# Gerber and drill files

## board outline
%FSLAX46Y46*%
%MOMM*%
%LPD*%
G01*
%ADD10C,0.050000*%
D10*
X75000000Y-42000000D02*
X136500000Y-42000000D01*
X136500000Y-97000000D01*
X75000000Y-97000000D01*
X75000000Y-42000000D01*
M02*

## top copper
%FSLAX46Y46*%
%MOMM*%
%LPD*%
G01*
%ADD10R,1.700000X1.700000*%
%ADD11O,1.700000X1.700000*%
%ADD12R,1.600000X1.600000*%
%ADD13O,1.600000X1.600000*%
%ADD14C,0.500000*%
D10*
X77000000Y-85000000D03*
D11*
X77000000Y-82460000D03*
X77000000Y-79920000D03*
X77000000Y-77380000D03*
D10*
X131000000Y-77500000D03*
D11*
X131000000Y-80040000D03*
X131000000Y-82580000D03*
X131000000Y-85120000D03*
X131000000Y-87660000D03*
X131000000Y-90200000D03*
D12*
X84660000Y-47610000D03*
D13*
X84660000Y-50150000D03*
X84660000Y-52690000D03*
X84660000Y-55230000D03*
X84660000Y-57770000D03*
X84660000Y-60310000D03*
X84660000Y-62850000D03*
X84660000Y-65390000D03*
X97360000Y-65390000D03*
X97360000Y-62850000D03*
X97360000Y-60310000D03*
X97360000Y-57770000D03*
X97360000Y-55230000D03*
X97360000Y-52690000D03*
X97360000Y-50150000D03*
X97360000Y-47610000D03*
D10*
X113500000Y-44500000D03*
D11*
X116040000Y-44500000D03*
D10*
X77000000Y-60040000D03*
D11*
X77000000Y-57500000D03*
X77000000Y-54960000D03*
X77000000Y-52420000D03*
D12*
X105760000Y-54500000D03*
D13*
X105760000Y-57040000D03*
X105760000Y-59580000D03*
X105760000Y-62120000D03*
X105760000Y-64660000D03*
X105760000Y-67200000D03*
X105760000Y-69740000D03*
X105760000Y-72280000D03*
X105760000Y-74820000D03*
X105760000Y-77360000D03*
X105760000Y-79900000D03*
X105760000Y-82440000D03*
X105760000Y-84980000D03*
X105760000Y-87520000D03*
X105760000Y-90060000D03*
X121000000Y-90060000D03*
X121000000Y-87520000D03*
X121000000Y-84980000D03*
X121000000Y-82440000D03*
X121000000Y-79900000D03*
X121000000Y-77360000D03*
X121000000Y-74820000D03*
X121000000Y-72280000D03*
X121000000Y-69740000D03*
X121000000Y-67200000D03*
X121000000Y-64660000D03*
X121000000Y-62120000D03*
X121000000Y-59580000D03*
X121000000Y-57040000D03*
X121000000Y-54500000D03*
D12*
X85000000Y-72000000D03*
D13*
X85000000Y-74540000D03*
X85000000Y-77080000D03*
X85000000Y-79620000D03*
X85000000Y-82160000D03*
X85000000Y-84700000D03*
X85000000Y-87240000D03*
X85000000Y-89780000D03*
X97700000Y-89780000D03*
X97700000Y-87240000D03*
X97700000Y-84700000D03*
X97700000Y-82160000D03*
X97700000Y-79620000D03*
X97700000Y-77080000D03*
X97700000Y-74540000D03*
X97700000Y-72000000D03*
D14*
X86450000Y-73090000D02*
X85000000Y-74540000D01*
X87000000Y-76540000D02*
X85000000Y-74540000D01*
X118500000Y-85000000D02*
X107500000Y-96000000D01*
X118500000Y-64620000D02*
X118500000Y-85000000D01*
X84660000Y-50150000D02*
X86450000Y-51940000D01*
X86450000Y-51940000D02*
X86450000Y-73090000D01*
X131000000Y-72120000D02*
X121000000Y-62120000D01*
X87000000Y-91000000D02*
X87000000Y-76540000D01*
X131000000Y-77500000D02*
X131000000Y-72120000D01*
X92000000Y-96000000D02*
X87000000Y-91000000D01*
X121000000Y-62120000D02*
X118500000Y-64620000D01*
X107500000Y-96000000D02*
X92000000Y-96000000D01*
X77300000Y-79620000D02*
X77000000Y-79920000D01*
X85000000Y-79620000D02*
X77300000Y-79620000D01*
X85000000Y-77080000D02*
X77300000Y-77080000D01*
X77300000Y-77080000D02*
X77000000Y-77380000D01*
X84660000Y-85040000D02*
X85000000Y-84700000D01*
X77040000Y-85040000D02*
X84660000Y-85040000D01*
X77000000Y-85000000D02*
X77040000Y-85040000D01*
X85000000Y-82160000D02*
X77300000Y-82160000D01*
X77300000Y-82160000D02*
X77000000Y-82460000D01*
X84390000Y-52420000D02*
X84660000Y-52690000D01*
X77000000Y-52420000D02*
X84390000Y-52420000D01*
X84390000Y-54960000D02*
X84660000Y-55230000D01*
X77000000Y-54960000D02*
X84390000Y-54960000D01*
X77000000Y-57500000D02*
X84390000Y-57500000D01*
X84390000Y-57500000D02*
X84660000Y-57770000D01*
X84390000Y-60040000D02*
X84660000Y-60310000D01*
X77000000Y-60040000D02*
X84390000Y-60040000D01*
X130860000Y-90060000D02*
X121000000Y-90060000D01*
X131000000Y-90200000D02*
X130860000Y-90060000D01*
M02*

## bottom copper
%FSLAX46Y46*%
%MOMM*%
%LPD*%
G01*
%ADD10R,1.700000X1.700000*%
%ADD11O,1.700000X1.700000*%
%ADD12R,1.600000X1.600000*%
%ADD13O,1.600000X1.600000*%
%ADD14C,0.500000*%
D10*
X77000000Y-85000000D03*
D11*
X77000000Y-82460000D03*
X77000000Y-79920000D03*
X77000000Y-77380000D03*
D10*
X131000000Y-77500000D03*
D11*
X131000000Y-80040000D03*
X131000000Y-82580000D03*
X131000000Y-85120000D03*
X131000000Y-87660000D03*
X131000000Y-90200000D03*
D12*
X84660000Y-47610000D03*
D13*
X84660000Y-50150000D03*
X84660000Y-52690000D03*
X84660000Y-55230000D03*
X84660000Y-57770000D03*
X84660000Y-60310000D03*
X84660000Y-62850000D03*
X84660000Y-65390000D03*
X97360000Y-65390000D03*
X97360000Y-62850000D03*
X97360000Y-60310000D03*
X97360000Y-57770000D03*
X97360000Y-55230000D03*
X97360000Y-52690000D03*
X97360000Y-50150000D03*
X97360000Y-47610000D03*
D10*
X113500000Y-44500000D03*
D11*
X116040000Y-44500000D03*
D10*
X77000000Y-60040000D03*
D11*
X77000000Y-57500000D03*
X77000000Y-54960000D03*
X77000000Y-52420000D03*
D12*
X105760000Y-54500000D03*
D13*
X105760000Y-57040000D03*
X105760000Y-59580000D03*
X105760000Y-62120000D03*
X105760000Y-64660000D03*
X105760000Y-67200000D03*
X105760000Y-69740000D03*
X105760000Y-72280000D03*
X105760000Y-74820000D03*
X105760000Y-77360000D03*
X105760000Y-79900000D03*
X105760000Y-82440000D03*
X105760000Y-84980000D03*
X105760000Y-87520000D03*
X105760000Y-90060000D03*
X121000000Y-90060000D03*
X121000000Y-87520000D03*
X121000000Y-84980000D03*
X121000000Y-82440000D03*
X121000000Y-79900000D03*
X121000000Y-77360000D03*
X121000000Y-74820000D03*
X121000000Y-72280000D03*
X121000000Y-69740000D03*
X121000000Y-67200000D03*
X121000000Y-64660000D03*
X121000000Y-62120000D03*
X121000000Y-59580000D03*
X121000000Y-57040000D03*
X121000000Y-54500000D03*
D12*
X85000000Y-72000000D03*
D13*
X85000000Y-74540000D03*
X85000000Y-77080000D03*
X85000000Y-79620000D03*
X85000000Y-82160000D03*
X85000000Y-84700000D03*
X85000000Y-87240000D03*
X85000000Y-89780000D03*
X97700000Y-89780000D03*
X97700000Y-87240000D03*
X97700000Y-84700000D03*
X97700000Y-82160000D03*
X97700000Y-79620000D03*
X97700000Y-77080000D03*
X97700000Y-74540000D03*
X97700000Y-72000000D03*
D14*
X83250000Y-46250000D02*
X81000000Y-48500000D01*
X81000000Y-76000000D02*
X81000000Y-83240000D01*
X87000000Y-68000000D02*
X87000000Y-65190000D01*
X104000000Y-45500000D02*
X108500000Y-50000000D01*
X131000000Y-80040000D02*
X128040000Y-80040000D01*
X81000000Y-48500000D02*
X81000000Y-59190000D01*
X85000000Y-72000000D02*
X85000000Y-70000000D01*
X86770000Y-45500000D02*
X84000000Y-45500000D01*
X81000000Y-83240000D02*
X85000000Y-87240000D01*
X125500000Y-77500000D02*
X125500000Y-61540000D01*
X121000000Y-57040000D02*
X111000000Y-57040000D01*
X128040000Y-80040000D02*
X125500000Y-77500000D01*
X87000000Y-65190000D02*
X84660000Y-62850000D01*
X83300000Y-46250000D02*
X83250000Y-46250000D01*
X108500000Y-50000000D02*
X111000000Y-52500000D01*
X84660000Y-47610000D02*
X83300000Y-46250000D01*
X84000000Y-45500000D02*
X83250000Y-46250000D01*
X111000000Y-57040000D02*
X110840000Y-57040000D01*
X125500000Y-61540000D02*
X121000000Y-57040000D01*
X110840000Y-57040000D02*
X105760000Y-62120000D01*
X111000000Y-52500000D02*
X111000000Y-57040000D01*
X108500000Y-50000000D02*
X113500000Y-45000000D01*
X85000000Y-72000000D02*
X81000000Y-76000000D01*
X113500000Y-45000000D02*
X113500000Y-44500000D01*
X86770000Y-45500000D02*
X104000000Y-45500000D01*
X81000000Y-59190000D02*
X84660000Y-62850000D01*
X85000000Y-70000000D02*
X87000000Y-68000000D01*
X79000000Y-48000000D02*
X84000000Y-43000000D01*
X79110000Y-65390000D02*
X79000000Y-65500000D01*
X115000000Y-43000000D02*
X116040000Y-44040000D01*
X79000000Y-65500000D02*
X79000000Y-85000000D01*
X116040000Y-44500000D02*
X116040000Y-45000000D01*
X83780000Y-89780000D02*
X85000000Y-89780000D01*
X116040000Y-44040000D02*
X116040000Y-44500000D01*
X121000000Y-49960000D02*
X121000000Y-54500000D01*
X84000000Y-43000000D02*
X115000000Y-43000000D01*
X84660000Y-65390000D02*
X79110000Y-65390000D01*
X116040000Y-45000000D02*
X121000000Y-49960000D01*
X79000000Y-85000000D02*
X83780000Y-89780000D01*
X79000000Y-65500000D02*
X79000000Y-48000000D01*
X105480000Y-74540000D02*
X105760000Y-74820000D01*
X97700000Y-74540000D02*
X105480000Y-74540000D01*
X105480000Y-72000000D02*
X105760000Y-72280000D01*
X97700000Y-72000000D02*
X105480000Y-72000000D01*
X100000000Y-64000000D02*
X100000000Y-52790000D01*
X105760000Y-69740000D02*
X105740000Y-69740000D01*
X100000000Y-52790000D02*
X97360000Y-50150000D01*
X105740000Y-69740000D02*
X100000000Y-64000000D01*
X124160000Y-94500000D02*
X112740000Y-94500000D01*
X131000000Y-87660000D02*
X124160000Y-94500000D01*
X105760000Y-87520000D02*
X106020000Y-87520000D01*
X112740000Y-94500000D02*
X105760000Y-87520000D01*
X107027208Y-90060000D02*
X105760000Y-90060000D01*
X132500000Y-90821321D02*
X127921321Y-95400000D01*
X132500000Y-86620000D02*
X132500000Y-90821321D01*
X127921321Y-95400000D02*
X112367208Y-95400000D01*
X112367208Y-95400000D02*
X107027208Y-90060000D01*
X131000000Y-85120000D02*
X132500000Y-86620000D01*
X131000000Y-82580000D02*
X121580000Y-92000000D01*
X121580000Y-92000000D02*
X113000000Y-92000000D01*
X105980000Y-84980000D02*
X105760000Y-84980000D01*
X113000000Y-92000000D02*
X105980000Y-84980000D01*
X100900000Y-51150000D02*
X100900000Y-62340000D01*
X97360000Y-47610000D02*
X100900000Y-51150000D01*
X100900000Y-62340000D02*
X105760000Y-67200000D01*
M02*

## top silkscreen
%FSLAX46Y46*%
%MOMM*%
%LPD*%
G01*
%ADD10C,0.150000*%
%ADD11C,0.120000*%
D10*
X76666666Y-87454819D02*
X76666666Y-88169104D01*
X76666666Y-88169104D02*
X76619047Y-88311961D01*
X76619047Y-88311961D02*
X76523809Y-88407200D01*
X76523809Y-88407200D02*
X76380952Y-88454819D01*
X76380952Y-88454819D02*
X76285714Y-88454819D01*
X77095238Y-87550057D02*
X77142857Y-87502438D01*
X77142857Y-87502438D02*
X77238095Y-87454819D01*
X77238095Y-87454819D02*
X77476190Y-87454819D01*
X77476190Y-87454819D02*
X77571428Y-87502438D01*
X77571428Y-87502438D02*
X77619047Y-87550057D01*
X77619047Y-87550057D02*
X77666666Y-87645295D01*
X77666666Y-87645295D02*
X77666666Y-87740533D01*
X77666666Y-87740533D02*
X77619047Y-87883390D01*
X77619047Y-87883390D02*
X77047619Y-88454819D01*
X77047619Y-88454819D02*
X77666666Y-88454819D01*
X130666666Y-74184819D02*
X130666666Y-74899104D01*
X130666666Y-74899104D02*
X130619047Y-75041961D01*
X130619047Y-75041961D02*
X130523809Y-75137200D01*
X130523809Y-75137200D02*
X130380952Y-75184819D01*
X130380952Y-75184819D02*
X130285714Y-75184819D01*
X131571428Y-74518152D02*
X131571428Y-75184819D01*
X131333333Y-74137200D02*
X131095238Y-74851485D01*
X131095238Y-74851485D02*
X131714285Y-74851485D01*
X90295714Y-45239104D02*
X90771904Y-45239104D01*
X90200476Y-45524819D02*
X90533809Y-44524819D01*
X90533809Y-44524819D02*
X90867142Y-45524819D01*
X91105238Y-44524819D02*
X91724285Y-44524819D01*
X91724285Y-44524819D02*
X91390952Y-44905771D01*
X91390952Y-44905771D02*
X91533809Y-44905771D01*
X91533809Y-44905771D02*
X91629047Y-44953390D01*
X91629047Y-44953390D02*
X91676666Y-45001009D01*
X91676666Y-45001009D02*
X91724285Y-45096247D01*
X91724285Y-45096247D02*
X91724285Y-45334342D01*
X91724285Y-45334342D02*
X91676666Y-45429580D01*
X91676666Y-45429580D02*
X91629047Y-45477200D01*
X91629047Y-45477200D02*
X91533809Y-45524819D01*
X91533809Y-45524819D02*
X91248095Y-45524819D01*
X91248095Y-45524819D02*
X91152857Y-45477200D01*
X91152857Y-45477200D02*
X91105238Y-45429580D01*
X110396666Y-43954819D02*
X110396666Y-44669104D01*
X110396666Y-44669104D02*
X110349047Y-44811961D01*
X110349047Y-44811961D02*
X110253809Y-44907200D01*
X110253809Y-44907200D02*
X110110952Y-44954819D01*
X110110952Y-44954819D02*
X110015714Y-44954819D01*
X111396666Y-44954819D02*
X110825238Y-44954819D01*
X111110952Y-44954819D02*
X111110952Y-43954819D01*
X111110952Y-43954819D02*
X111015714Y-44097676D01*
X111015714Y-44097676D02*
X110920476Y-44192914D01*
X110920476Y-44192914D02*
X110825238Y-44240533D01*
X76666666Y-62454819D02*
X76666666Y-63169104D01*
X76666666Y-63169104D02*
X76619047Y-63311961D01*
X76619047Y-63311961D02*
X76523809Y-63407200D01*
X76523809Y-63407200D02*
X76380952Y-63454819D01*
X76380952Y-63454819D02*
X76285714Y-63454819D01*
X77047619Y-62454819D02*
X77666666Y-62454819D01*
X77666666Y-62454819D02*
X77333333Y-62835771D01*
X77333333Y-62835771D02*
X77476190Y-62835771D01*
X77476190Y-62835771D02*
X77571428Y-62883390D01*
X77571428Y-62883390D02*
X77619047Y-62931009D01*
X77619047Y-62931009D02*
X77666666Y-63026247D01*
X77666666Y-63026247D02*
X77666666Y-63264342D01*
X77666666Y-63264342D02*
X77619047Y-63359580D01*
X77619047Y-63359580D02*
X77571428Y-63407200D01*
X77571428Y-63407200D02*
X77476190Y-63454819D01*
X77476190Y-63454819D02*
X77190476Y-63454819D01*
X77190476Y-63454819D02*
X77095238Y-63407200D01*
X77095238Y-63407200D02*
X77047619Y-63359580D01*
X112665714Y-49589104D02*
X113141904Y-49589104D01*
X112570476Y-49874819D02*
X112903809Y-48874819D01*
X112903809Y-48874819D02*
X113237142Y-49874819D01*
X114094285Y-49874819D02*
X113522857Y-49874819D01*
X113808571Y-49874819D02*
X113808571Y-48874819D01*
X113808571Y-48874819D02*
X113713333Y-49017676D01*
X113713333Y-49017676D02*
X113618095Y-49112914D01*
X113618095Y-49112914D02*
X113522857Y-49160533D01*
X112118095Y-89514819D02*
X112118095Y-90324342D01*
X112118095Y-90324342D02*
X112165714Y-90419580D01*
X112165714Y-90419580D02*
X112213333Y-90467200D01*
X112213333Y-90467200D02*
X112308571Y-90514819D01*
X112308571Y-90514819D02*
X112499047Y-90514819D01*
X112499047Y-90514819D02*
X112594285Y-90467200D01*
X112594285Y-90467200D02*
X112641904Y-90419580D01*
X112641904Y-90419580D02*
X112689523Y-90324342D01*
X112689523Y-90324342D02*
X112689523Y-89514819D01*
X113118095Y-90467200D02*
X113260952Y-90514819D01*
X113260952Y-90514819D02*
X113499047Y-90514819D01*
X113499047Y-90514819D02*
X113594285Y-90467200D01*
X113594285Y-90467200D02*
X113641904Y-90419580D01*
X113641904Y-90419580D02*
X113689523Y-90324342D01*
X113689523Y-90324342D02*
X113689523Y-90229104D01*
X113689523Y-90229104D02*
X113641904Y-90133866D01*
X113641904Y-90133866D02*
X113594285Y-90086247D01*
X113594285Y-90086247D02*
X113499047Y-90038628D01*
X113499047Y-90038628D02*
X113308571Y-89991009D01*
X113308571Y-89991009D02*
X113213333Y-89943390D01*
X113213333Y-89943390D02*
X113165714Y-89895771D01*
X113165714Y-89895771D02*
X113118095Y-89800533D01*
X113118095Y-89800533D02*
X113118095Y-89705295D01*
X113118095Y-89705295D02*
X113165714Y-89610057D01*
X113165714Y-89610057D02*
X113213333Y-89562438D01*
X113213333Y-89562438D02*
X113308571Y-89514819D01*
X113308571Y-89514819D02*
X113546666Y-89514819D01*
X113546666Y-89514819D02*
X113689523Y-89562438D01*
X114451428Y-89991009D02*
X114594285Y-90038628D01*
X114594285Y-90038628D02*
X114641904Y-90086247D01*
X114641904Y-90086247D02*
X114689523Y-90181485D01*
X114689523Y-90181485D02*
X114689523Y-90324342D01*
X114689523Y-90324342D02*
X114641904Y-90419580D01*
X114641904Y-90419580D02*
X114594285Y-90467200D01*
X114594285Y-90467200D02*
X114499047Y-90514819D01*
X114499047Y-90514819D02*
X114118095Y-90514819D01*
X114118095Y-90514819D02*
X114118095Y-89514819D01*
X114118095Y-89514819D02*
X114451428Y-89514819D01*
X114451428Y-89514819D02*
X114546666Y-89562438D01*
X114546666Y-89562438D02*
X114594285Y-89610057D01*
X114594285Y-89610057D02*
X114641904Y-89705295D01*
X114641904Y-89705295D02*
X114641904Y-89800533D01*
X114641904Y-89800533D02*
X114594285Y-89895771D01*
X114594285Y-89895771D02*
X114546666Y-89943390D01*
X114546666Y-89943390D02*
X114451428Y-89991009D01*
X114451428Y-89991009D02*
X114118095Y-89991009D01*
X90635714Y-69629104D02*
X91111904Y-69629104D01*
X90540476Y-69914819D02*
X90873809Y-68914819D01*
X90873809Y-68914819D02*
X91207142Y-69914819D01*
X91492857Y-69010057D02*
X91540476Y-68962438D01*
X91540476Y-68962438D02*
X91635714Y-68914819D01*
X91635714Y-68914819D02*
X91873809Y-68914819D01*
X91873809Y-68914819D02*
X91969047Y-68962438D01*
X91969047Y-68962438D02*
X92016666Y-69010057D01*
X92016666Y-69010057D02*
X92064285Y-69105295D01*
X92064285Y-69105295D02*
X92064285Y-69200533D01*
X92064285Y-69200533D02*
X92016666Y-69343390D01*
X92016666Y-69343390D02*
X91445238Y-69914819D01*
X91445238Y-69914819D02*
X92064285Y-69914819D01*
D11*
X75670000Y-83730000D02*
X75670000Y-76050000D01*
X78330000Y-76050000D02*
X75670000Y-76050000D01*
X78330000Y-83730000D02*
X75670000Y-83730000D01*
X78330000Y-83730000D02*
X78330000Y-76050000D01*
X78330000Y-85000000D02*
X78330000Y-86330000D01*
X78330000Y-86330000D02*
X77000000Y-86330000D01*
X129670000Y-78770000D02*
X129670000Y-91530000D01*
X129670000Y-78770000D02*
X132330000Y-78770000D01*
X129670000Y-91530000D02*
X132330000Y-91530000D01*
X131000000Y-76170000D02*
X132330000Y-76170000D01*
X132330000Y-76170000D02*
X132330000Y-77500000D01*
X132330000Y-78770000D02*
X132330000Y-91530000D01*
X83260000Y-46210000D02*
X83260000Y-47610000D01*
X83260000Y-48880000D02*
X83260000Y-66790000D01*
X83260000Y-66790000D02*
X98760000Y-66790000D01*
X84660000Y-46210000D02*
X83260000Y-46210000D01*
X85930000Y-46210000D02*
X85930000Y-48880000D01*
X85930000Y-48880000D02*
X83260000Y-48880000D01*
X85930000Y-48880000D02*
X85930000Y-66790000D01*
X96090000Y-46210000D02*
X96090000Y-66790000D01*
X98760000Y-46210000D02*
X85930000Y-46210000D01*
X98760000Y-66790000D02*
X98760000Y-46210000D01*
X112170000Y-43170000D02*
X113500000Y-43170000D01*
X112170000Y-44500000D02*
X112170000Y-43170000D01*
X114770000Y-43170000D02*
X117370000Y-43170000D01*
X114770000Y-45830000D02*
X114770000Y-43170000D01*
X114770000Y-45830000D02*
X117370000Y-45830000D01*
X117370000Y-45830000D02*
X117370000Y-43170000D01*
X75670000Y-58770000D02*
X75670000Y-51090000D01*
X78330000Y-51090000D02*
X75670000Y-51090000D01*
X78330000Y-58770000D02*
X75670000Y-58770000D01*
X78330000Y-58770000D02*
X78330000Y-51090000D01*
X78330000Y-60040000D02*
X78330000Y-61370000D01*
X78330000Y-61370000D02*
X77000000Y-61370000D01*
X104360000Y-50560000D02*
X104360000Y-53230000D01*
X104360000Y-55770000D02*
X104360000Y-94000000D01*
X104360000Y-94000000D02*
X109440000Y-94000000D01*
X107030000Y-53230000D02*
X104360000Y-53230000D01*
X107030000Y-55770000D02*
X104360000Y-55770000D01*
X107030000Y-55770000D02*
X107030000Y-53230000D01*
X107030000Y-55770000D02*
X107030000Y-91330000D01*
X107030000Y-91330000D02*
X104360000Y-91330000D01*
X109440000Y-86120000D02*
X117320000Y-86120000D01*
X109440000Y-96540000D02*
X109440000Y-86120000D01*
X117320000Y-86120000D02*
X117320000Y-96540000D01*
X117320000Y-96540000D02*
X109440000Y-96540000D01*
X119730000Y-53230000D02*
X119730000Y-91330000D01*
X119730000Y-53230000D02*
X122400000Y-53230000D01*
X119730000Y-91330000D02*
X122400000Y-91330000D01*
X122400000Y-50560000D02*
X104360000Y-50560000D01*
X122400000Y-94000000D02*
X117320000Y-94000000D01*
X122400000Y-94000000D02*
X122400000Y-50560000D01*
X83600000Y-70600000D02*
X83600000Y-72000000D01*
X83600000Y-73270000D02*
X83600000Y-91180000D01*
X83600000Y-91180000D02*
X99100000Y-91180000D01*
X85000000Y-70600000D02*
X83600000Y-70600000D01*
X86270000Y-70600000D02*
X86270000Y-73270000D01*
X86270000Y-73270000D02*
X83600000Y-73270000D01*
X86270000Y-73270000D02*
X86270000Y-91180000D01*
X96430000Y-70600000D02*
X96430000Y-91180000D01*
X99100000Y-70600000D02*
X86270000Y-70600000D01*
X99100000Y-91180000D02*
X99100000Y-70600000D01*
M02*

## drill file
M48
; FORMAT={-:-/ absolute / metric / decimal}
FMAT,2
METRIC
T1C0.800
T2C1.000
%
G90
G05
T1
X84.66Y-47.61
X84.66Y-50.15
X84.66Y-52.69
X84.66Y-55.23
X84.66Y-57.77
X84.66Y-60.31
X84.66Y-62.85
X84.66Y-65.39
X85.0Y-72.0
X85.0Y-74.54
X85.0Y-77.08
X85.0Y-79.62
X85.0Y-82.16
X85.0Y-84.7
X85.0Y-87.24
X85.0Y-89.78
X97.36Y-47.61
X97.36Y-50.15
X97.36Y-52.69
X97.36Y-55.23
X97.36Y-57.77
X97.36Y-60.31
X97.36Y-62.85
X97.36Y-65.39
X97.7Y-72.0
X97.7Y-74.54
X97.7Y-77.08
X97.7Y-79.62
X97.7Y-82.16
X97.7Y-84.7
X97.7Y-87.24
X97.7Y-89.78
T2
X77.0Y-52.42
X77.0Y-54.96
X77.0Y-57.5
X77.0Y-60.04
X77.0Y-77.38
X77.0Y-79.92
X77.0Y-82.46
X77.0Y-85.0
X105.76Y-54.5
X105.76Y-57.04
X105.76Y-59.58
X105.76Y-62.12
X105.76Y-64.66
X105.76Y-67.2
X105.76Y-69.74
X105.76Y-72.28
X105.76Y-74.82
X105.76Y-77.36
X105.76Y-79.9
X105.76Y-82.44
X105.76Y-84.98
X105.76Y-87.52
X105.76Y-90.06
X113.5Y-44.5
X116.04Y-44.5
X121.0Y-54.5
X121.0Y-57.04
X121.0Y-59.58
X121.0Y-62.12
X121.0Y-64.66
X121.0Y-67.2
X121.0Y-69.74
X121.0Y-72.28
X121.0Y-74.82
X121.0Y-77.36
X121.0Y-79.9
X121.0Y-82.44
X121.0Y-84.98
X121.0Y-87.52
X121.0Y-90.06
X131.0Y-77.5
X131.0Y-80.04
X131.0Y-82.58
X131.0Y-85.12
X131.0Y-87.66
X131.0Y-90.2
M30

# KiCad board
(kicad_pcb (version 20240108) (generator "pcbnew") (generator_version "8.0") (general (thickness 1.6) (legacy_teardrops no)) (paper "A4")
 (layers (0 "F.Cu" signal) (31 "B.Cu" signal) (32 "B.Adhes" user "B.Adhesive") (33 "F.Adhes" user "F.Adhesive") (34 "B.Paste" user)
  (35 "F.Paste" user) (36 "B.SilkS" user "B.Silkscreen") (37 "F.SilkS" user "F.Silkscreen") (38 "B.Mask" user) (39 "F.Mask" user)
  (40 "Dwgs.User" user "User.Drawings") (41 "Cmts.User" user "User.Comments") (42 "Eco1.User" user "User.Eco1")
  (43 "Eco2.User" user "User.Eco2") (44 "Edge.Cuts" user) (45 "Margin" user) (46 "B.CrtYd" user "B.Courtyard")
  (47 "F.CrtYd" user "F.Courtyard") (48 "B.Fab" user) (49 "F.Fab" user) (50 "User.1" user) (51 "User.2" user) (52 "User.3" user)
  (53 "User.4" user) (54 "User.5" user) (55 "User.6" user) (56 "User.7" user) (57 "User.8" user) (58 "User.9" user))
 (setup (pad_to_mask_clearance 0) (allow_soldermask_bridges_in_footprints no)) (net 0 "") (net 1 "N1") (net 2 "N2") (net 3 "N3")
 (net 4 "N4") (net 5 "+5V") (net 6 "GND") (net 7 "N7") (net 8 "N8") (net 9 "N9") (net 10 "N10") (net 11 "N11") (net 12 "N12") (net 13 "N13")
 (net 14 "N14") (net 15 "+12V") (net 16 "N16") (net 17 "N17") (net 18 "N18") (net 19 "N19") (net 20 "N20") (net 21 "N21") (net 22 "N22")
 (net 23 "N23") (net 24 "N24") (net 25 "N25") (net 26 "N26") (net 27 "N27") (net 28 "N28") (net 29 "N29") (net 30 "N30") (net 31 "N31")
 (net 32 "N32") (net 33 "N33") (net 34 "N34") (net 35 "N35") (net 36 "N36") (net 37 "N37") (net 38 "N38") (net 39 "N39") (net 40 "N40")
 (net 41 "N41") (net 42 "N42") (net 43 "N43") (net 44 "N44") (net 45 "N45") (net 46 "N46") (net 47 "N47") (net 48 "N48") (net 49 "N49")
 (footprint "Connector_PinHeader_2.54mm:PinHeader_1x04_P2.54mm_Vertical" (layer "F.Cu") (at 77 85 180)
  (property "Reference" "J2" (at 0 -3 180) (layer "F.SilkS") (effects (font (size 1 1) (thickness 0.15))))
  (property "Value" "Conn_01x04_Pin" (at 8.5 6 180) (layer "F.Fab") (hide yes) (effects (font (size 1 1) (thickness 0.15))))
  (fp_line (start 1.33 1.27) (end 1.33 8.95) (stroke (width 0.12) (type solid)) (layer "F.SilkS"))
  (fp_line (start -1.33 8.95) (end 1.33 8.95) (stroke (width 0.12) (type solid)) (layer "F.SilkS"))
  (fp_line (start -1.33 1.27) (end 1.33 1.27) (stroke (width 0.12) (type solid)) (layer "F.SilkS"))
  (fp_line (start -1.33 1.27) (end -1.33 8.95) (stroke (width 0.12) (type solid)) (layer "F.SilkS"))
  (fp_line (start -1.33 0) (end -1.33 -1.33) (stroke (width 0.12) (type solid)) (layer "F.SilkS"))
  (fp_line (start -1.33 -1.33) (end 0 -1.33) (stroke (width 0.12) (type solid)) (layer "F.SilkS"))
  (pad "1" thru_hole rect (at 0 0 180) (size 1.7 1.7) (drill 1) (layers "*.Cu" "*.Mask") (remove_unused_layers no) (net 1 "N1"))
  (pad "2" thru_hole oval (at 0 2.54 180) (size 1.7 1.7) (drill 1) (layers "*.Cu" "*.Mask") (remove_unused_layers no) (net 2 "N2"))
  (pad "3" thru_hole oval (at 0 5.08 180) (size 1.7 1.7) (drill 1) (layers "*.Cu" "*.Mask") (remove_unused_layers no) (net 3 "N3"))
  (pad "4" thru_hole oval (at 0 7.62 180) (size 1.7 1.7) (drill 1) (layers "*.Cu" "*.Mask") (remove_unused_layers no) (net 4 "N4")))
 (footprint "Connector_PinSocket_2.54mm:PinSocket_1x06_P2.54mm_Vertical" (layer "F.Cu") (at 131 77.5)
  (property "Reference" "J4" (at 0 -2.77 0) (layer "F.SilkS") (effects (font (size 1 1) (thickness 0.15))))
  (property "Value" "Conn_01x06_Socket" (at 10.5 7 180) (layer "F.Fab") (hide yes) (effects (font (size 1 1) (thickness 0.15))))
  (fp_line (start -1.33 1.27) (end -1.33 14.03) (stroke (width 0.12) (type solid)) (layer "F.SilkS"))
  (fp_line (start -1.33 1.27) (end 1.33 1.27) (stroke (width 0.12) (type solid)) (layer "F.SilkS"))
  (fp_line (start -1.33 14.03) (end 1.33 14.03) (stroke (width 0.12) (type solid)) (layer "F.SilkS"))
  (fp_line (start 0 -1.33) (end 1.33 -1.33) (stroke (width 0.12) (type solid)) (layer "F.SilkS"))
  (fp_line (start 1.33 -1.33) (end 1.33 0) (stroke (width 0.12) (type solid)) (layer "F.SilkS"))
  (fp_line (start 1.33 1.27) (end 1.33 14.03) (stroke (width 0.12) (type solid)) (layer "F.SilkS"))
  (pad "1" thru_hole rect (at 0 0) (size 1.7 1.7) (drill 1) (layers "*.Cu" "*.Mask") (remove_unused_layers no) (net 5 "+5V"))
  (pad "2" thru_hole oval (at 0 2.54) (size 1.7 1.7) (drill 1) (layers "*.Cu" "*.Mask") (remove_unused_layers no) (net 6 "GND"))
  (pad "3" thru_hole oval (at 0 5.08) (size 1.7 1.7) (drill 1) (layers "*.Cu" "*.Mask") (remove_unused_layers no) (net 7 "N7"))
  (pad "4" thru_hole oval (at 0 7.62) (size 1.7 1.7) (drill 1) (layers "*.Cu" "*.Mask") (remove_unused_layers no) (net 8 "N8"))
  (pad "5" thru_hole oval (at 0 10.16) (size 1.7 1.7) (drill 1) (layers "*.Cu" "*.Mask") (remove_unused_layers no) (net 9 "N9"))
  (pad "6" thru_hole oval (at 0 12.7) (size 1.7 1.7) (drill 1) (layers "*.Cu" "*.Mask") (remove_unused_layers no) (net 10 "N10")))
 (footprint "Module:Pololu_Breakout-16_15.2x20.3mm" (layer "F.Cu") (at 84.66 47.61)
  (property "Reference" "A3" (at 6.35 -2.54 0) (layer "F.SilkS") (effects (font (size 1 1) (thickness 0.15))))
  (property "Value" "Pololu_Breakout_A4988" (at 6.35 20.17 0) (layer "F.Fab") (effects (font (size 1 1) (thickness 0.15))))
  (fp_line (start -1.4 -1.4) (end -1.4 0) (stroke (width 0.12) (type solid)) (layer "F.SilkS"))
  (fp_line (start -1.4 1.27) (end -1.4 19.18) (stroke (width 0.12) (type solid)) (layer "F.SilkS"))
  (fp_line (start -1.4 19.18) (end 14.1 19.18) (stroke (width 0.12) (type solid)) (layer "F.SilkS"))
  (fp_line (start 0 -1.4) (end -1.4 -1.4) (stroke (width 0.12) (type solid)) (layer "F.SilkS"))
  (fp_line (start 1.27 -1.4) (end 1.27 1.27) (stroke (width 0.12) (type solid)) (layer "F.SilkS"))
  (fp_line (start 1.27 1.27) (end -1.4 1.27) (stroke (width 0.12) (type solid)) (layer "F.SilkS"))
  (fp_line (start 1.27 1.27) (end 1.27 19.18) (stroke (width 0.12) (type solid)) (layer "F.SilkS"))
  (fp_line (start 11.43 -1.4) (end 11.43 19.18) (stroke (width 0.12) (type solid)) (layer "F.SilkS"))
  (fp_line (start 14.1 -1.4) (end 1.27 -1.4) (stroke (width 0.12) (type solid)) (layer "F.SilkS"))
  (fp_line (start 14.1 19.18) (end 14.1 -1.4) (stroke (width 0.12) (type solid)) (layer "F.SilkS"))
  (pad "1" thru_hole rect (at 0 0) (size 1.6 1.6) (drill 0.8) (layers "*.Cu" "*.Mask") (remove_unused_layers no) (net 6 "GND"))
  (pad "2" thru_hole oval (at 0 2.54) (size 1.6 1.6) (drill 0.8) (layers "*.Cu" "*.Mask") (remove_unused_layers no) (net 5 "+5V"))
  (pad "3" thru_hole oval (at 0 5.08) (size 1.6 1.6) (drill 0.8) (layers "*.Cu" "*.Mask") (remove_unused_layers no) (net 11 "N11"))
  (pad "4" thru_hole oval (at 0 7.62) (size 1.6 1.6) (drill 0.8) (layers "*.Cu" "*.Mask") (remove_unused_layers no) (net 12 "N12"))
  (pad "5" thru_hole oval (at 0 10.16) (size 1.6 1.6) (drill 0.8) (layers "*.Cu" "*.Mask") (remove_unused_layers no) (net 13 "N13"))
  (pad "6" thru_hole oval (at 0 12.7) (size 1.6 1.6) (drill 0.8) (layers "*.Cu" "*.Mask") (remove_unused_layers no) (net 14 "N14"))
  (pad "7" thru_hole oval (at 0 15.24) (size 1.6 1.6) (drill 0.8) (layers "*.Cu" "*.Mask") (remove_unused_layers no) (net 6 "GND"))
  (pad "8" thru_hole oval (at 0 17.78) (size 1.6 1.6) (drill 0.8) (layers "*.Cu" "*.Mask") (remove_unused_layers no) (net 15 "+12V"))
  (pad "9" thru_hole oval (at 12.7 17.78) (size 1.6 1.6) (drill 0.8) (layers "*.Cu" "*.Mask") (remove_unused_layers no) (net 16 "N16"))
  (pad "10" thru_hole oval (at 12.7 15.24) (size 1.6 1.6) (drill 0.8) (layers "*.Cu" "*.Mask") (remove_unused_layers no) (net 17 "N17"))
  (pad "11" thru_hole oval (at 12.7 12.7) (size 1.6 1.6) (drill 0.8) (layers "*.Cu" "*.Mask") (remove_unused_layers no) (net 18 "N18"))
  (pad "12" thru_hole oval (at 12.7 10.16) (size 1.6 1.6) (drill 0.8) (layers "*.Cu" "*.Mask") (remove_unused_layers no) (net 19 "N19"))
  (pad "13" thru_hole oval (at 12.7 7.62) (size 1.6 1.6) (drill 0.8) (layers "*.Cu" "*.Mask") (remove_unused_layers no) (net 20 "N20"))
  (pad "14" thru_hole oval (at 12.7 5.08) (size 1.6 1.6) (drill 0.8) (layers "*.Cu" "*.Mask") (remove_unused_layers no) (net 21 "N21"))
  (pad "15" thru_hole oval (at 12.7 2.54) (size 1.6 1.6) (drill 0.8) (layers "*.Cu" "*.Mask") (remove_unused_layers no) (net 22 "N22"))
  (pad "16" thru_hole oval (at 12.7 0) (size 1.6 1.6) (drill 0.8) (layers "*.Cu" "*.Mask") (remove_unused_layers no) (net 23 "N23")))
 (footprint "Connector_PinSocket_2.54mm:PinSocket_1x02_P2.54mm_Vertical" (layer "F.Cu") (at 113.5 44.5 90)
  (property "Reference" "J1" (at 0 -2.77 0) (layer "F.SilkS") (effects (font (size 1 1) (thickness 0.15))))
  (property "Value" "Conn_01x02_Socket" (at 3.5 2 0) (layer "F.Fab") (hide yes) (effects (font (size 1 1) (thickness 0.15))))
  (fp_line (start 1.33 -1.33) (end 1.33 0) (stroke (width 0.12) (type solid)) (layer "F.SilkS"))
  (fp_line (start 0 -1.33) (end 1.33 -1.33) (stroke (width 0.12) (type solid)) (layer "F.SilkS"))
  (fp_line (start 1.33 1.27) (end 1.33 3.87) (stroke (width 0.12) (type solid)) (layer "F.SilkS"))
  (fp_line (start -1.33 1.27) (end 1.33 1.27) (stroke (width 0.12) (type solid)) (layer "F.SilkS"))
  (fp_line (start -1.33 1.27) (end -1.33 3.87) (stroke (width 0.12) (type solid)) (layer "F.SilkS"))
  (fp_line (start -1.33 3.87) (end 1.33 3.87) (stroke (width 0.12) (type solid)) (layer "F.SilkS"))
  (pad "1" thru_hole rect (at 0 0 90) (size 1.7 1.7) (drill 1) (layers "*.Cu" "*.Mask") (remove_unused_layers no) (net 6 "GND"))
  (pad "2" thru_hole oval (at 0 2.54 90) (size 1.7 1.7) (drill 1) (layers "*.Cu" "*.Mask") (remove_unused_layers no) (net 15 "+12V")))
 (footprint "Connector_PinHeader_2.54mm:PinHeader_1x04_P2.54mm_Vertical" (layer "F.Cu") (at 77 60.04 180)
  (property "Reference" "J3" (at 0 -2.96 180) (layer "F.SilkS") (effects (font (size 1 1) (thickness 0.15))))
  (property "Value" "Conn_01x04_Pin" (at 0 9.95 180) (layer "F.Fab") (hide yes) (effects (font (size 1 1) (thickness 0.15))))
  (fp_line (start 1.33 1.27) (end 1.33 8.95) (stroke (width 0.12) (type solid)) (layer "F.SilkS"))
  (fp_line (start -1.33 8.95) (end 1.33 8.95) (stroke (width 0.12) (type solid)) (layer "F.SilkS"))
  (fp_line (start -1.33 1.27) (end 1.33 1.27) (stroke (width 0.12) (type solid)) (layer "F.SilkS"))
  (fp_line (start -1.33 1.27) (end -1.33 8.95) (stroke (width 0.12) (type solid)) (layer "F.SilkS"))
  (fp_line (start -1.33 0) (end -1.33 -1.33) (stroke (width 0.12) (type solid)) (layer "F.SilkS"))
  (fp_line (start -1.33 -1.33) (end 0 -1.33) (stroke (width 0.12) (type solid)) (layer "F.SilkS"))
  (pad "1" thru_hole rect (at 0 0 180) (size 1.7 1.7) (drill 1) (layers "*.Cu" "*.Mask") (remove_unused_layers no) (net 14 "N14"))
  (pad "2" thru_hole oval (at 0 2.54 180) (size 1.7 1.7) (drill 1) (layers "*.Cu" "*.Mask") (remove_unused_layers no) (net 13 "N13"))
  (pad "3" thru_hole oval (at 0 5.08 180) (size 1.7 1.7) (drill 1) (layers "*.Cu" "*.Mask") (remove_unused_layers no) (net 12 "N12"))
  (pad "4" thru_hole oval (at 0 7.62 180) (size 1.7 1.7) (drill 1) (layers "*.Cu" "*.Mask") (remove_unused_layers no) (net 11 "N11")))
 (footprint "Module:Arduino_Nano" (layer "F.Cu") (at 105.76 54.5)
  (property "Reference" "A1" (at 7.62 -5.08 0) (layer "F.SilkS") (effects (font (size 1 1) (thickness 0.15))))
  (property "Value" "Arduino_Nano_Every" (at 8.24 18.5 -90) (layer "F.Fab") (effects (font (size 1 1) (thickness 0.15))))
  (fp_line (start -1.4 -3.94) (end -1.4 -1.27) (stroke (width 0.12) (type solid)) (layer "F.SilkS"))
  (fp_line (start -1.4 1.27) (end -1.4 39.5) (stroke (width 0.12) (type solid)) (layer "F.SilkS"))
  (fp_line (start -1.4 39.5) (end 3.68 39.5) (stroke (width 0.12) (type solid)) (layer "F.SilkS"))
  (fp_line (start 1.27 -1.27) (end -1.4 -1.27) (stroke (width 0.12) (type solid)) (layer "F.SilkS"))
  (fp_line (start 1.27 1.27) (end -1.4 1.27) (stroke (width 0.12) (type solid)) (layer "F.SilkS"))
  (fp_line (start 1.27 1.27) (end 1.27 -1.27) (stroke (width 0.12) (type solid)) (layer "F.SilkS"))
  (fp_line (start 1.27 1.27) (end 1.27 36.83) (stroke (width 0.12) (type solid)) (layer "F.SilkS"))
  (fp_line (start 1.27 36.83) (end -1.4 36.83) (stroke (width 0.12) (type solid)) (layer "F.SilkS"))
  (fp_line (start 3.68 31.62) (end 11.56 31.62) (stroke (width 0.12) (type solid)) (layer "F.SilkS"))
  (fp_line (start 3.68 42.04) (end 3.68 31.62) (stroke (width 0.12) (type solid)) (layer "F.SilkS"))
  (fp_line (start 11.56 31.62) (end 11.56 42.04) (stroke (width 0.12) (type solid)) (layer "F.SilkS"))
  (fp_line (start 11.56 42.04) (end 3.68 42.04) (stroke (width 0.12) (type solid)) (layer "F.SilkS"))
  (fp_line (start 13.97 -1.27) (end 13.97 36.83) (stroke (width 0.12) (type solid)) (layer "F.SilkS"))
  (fp_line (start 13.97 -1.27) (end 16.64 -1.27) (stroke (width 0.12) (type solid)) (layer "F.SilkS"))
  (fp_line (start 13.97 36.83) (end 16.64 36.83) (stroke (width 0.12) (type solid)) (layer "F.SilkS"))
  (fp_line (start 16.64 -3.94) (end -1.4 -3.94) (stroke (width 0.12) (type solid)) (layer "F.SilkS"))
  (fp_line (start 16.64 39.5) (end 11.56 39.5) (stroke (width 0.12) (type solid)) (layer "F.SilkS"))
  (fp_line (start 16.64 39.5) (end 16.64 -3.94) (stroke (width 0.12) (type solid)) (layer "F.SilkS"))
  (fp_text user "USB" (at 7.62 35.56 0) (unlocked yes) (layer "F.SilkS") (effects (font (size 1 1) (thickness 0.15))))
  (pad "1" thru_hole rect (at 0 0) (size 1.6 1.6) (drill 1) (layers "*.Cu" "*.Mask") (remove_unused_layers no) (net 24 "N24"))
  (pad "2" thru_hole oval (at 0 2.54) (size 1.6 1.6) (drill 1) (layers "*.Cu" "*.Mask") (remove_unused_layers no) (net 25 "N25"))
  (pad "3" thru_hole oval (at 0 5.08) (size 1.6 1.6) (drill 1) (layers "*.Cu" "*.Mask") (remove_unused_layers no) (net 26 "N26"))
  (pad "4" thru_hole oval (at 0 7.62) (size 1.6 1.6) (drill 1) (layers "*.Cu" "*.Mask") (remove_unused_layers no) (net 6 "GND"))
  (pad "5" thru_hole oval (at 0 10.16) (size 1.6 1.6) (drill 1) (layers "*.Cu" "*.Mask") (remove_unused_layers no) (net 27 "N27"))
  (pad "6" thru_hole oval (at 0 12.7) (size 1.6 1.6) (drill 1) (layers "*.Cu" "*.Mask") (remove_unused_layers no) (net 23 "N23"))
  (pad "7" thru_hole oval (at 0 15.24) (size 1.6 1.6) (drill 1) (layers "*.Cu" "*.Mask") (remove_unused_layers no) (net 22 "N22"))
  (pad "8" thru_hole oval (at 0 17.78) (size 1.6 1.6) (drill 1) (layers "*.Cu" "*.Mask") (remove_unused_layers no) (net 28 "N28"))
  (pad "9" thru_hole oval (at 0 20.32) (size 1.6 1.6) (drill 1) (layers "*.Cu" "*.Mask") (remove_unused_layers no) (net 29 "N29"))
  (pad "10" thru_hole oval (at 0 22.86) (size 1.6 1.6) (drill 1) (layers "*.Cu" "*.Mask") (remove_unused_layers no) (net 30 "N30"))
  (pad "11" thru_hole oval (at 0 25.4) (size 1.6 1.6) (drill 1) (layers "*.Cu" "*.Mask") (remove_unused_layers no) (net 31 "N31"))
  (pad "12" thru_hole oval (at 0 27.94) (size 1.6 1.6) (drill 1) (layers "*.Cu" "*.Mask") (remove_unused_layers no) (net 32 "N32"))
  (pad "13" thru_hole oval (at 0 30.48) (size 1.6 1.6) (drill 1) (layers "*.Cu" "*.Mask") (remove_unused_layers no) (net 7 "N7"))
  (pad "14" thru_hole oval (at 0 33.02) (size 1.6 1.6) (drill 1) (layers "*.Cu" "*.Mask") (remove_unused_layers no) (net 9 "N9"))
  (pad "15" thru_hole oval (at 0 35.56) (size 1.6 1.6) (drill 1) (layers "*.Cu" "*.Mask") (remove_unused_layers no) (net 8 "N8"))
  (pad "16" thru_hole oval (at 15.24 35.56) (size 1.6 1.6) (drill 1) (layers "*.Cu" "*.Mask") (remove_unused_layers no) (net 10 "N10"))
  (pad "17" thru_hole oval (at 15.24 33.02) (size 1.6 1.6) (drill 1) (layers "*.Cu" "*.Mask") (remove_unused_layers no) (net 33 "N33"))
  (pad "18" thru_hole oval (at 15.24 30.48) (size 1.6 1.6) (drill 1) (layers "*.Cu" "*.Mask") (remove_unused_layers no) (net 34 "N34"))
  (pad "19" thru_hole oval (at 15.24 27.94) (size 1.6 1.6) (drill 1) (layers "*.Cu" "*.Mask") (remove_unused_layers no) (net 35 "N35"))
  (pad "20" thru_hole oval (at 15.24 25.4) (size 1.6 1.6) (drill 1) (layers "*.Cu" "*.Mask") (remove_unused_layers no) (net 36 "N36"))
  (pad "21" thru_hole oval (at 15.24 22.86) (size 1.6 1.6) (drill 1) (layers "*.Cu" "*.Mask") (remove_unused_layers no) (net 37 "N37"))
  (pad "22" thru_hole oval (at 15.24 20.32) (size 1.6 1.6) (drill 1) (layers "*.Cu" "*.Mask") (remove_unused_layers no) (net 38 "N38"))
  (pad "23" thru_hole oval (at 15.24 17.78) (size 1.6 1.6) (drill 1) (layers "*.Cu" "*.Mask") (remove_unused_layers no) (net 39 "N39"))
  (pad "24" thru_hole oval (at 15.24 15.24) (size 1.6 1.6) (drill 1) (layers "*.Cu" "*.Mask") (remove_unused_layers no) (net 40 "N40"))
  (pad "25" thru_hole oval (at 15.24 12.7) (size 1.6 1.6) (drill 1) (layers "*.Cu" "*.Mask") (remove_unused_layers no) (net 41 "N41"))
  (pad "26" thru_hole oval (at 15.24 10.16) (size 1.6 1.6) (drill 1) (layers "*.Cu" "*.Mask") (remove_unused_layers no) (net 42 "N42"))
  (pad "27" thru_hole oval (at 15.24 7.62) (size 1.6 1.6) (drill 1) (layers "*.Cu" "*.Mask") (remove_unused_layers no) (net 5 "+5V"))
  (pad "28" thru_hole oval (at 15.24 5.08) (size 1.6 1.6) (drill 1) (layers "*.Cu" "*.Mask") (remove_unused_layers no) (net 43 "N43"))
  (pad "29" thru_hole oval (at 15.24 2.54) (size 1.6 1.6) (drill 1) (layers "*.Cu" "*.Mask") (remove_unused_layers no) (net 6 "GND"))
  (pad "30" thru_hole oval (at 15.24 0) (size 1.6 1.6) (drill 1) (layers "*.Cu" "*.Mask") (remove_unused_layers no) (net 15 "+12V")))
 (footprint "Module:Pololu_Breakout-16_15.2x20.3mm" (layer "F.Cu") (at 85 72)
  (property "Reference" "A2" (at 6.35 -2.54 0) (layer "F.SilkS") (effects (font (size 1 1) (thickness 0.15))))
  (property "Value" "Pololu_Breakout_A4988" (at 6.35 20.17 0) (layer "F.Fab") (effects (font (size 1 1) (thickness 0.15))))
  (fp_line (start -1.4 -1.4) (end -1.4 0) (stroke (width 0.12) (type solid)) (layer "F.SilkS"))
  (fp_line (start -1.4 1.27) (end -1.4 19.18) (stroke (width 0.12) (type solid)) (layer "F.SilkS"))
  (fp_line (start -1.4 19.18) (end 14.1 19.18) (stroke (width 0.12) (type solid)) (layer "F.SilkS"))
  (fp_line (start 0 -1.4) (end -1.4 -1.4) (stroke (width 0.12) (type solid)) (layer "F.SilkS"))
  (fp_line (start 1.27 -1.4) (end 1.27 1.27) (stroke (width 0.12) (type solid)) (layer "F.SilkS"))
  (fp_line (start 1.27 1.27) (end -1.4 1.27) (stroke (width 0.12) (type solid)) (layer "F.SilkS"))
  (fp_line (start 1.27 1.27) (end 1.27 19.18) (stroke (width 0.12) (type solid)) (layer "F.SilkS"))
  (fp_line (start 11.43 -1.4) (end 11.43 19.18) (stroke (width 0.12) (type solid)) (layer "F.SilkS"))
  (fp_line (start 14.1 -1.4) (end 1.27 -1.4) (stroke (width 0.12) (type solid)) (layer "F.SilkS"))
  (fp_line (start 14.1 19.18) (end 14.1 -1.4) (stroke (width 0.12) (type solid)) (layer "F.SilkS"))
  (pad "1" thru_hole rect (at 0 0) (size 1.6 1.6) (drill 0.8) (layers "*.Cu" "*.Mask") (remove_unused_layers no) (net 6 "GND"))
  (pad "2" thru_hole oval (at 0 2.54) (size 1.6 1.6) (drill 0.8) (layers "*.Cu" "*.Mask") (remove_unused_layers no) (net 5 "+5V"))
  (pad "3" thru_hole oval (at 0 5.08) (size 1.6 1.6) (drill 0.8) (layers "*.Cu" "*.Mask") (remove_unused_layers no) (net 4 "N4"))
  (pad "4" thru_hole oval (at 0 7.62) (size 1.6 1.6) (drill 0.8) (layers "*.Cu" "*.Mask") (remove_unused_layers no) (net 3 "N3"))
  (pad "5" thru_hole oval (at 0 10.16) (size 1.6 1.6) (drill 0.8) (layers "*.Cu" "*.Mask") (remove_unused_layers no) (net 2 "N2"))
  (pad "6" thru_hole oval (at 0 12.7) (size 1.6 1.6) (drill 0.8) (layers "*.Cu" "*.Mask") (remove_unused_layers no) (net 1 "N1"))
  (pad "7" thru_hole oval (at 0 15.24) (size 1.6 1.6) (drill 0.8) (layers "*.Cu" "*.Mask") (remove_unused_layers no) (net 6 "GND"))
  (pad "8" thru_hole oval (at 0 17.78) (size 1.6 1.6) (drill 0.8) (layers "*.Cu" "*.Mask") (remove_unused_layers no) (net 15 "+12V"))
  (pad "9" thru_hole oval (at 12.7 17.78) (size 1.6 1.6) (drill 0.8) (layers "*.Cu" "*.Mask") (remove_unused_layers no) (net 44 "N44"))
  (pad "10" thru_hole oval (at 12.7 15.24) (size 1.6 1.6) (drill 0.8) (layers "*.Cu" "*.Mask") (remove_unused_layers no) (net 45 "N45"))
  (pad "11" thru_hole oval (at 12.7 12.7) (size 1.6 1.6) (drill 0.8) (layers "*.Cu" "*.Mask") (remove_unused_layers no) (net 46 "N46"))
  (pad "12" thru_hole oval (at 12.7 10.16) (size 1.6 1.6) (drill 0.8) (layers "*.Cu" "*.Mask") (remove_unused_layers no) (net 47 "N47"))
  (pad "13" thru_hole oval (at 12.7 7.62) (size 1.6 1.6) (drill 0.8) (layers "*.Cu" "*.Mask") (remove_unused_layers no) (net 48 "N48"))
  (pad "14" thru_hole oval (at 12.7 5.08) (size 1.6 1.6) (drill 0.8) (layers "*.Cu" "*.Mask") (remove_unused_layers no) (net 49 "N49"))
  (pad "15" thru_hole oval (at 12.7 2.54) (size 1.6 1.6) (drill 0.8) (layers "*.Cu" "*.Mask") (remove_unused_layers no) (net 29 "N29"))
  (pad "16" thru_hole oval (at 12.7 0) (size 1.6 1.6) (drill 0.8) (layers "*.Cu" "*.Mask") (remove_unused_layers no) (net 28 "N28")))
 (gr_rect (start 75 42) (end 136.5 97) (stroke (width 0.05) (type default)) (fill none) (layer "Edge.Cuts"))
 (segment (start 83.25 46.25) (end 81 48.5) (width 0.5) (layer "B.Cu") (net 6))
 (segment (start 81 76) (end 81 83.24) (width 0.5) (layer "B.Cu") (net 6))
 (segment (start 87 68) (end 87 65.19) (width 0.5) (layer "B.Cu") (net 6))
 (segment (start 104 45.5) (end 108.5 50) (width 0.5) (layer "B.Cu") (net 6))
 (segment (start 131 80.04) (end 128.04 80.04) (width 0.5) (layer "B.Cu") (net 6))
 (segment (start 81 48.5) (end 81 59.19) (width 0.5) (layer "B.Cu") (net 6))
 (segment (start 85 72) (end 85 70) (width 0.5) (layer "B.Cu") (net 6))
 (segment (start 86.77 45.5) (end 84 45.5) (width 0.5) (layer "B.Cu") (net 6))
 (segment (start 81 83.24) (end 85 87.24) (width 0.5) (layer "B.Cu") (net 6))
 (segment (start 125.5 77.5) (end 125.5 61.54) (width 0.5) (layer "B.Cu") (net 6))
 (segment (start 121 57.04) (end 111 57.04) (width 0.5) (layer "B.Cu") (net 6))
 (segment (start 128.04 80.04) (end 125.5 77.5) (width 0.5) (layer "B.Cu") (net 6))
 (segment (start 87 65.19) (end 84.66 62.85) (width 0.5) (layer "B.Cu") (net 6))
 (segment (start 83.3 46.25) (end 83.25 46.25) (width 0.5) (layer "B.Cu") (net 6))
 (segment (start 108.5 50) (end 111 52.5) (width 0.5) (layer "B.Cu") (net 6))
 (segment (start 84.66 47.61) (end 83.3 46.25) (width 0.5) (layer "B.Cu") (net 6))
 (segment (start 84 45.5) (end 83.25 46.25) (width 0.5) (layer "B.Cu") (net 6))
 (segment (start 111 57.04) (end 110.84 57.04) (width 0.5) (layer "B.Cu") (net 6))
 (segment (start 125.5 61.54) (end 121 57.04) (width 0.5) (layer "B.Cu") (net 6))
 (segment (start 110.84 57.04) (end 105.76 62.12) (width 0.5) (layer "B.Cu") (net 6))
 (segment (start 111 52.5) (end 111 57.04) (width 0.5) (layer "B.Cu") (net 6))
 (segment (start 108.5 50) (end 113.5 45) (width 0.5) (layer "B.Cu") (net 6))
 (segment (start 85 72) (end 81 76) (width 0.5) (layer "B.Cu") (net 6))
 (segment (start 113.5 45) (end 113.5 44.5) (width 0.5) (layer "B.Cu") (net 6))
 (segment (start 86.77 45.5) (end 104 45.5) (width 0.5) (layer "B.Cu") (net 6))
 (segment (start 81 59.19) (end 84.66 62.85) (width 0.5) (layer "B.Cu") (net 6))
 (segment (start 85 70) (end 87 68) (width 0.5) (layer "B.Cu") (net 6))
 (segment (start 79 48) (end 84 43) (width 0.5) (layer "B.Cu") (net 15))
 (segment (start 79.11 65.39) (end 79 65.5) (width 0.5) (layer "B.Cu") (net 15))
 (segment (start 115 43) (end 116.04 44.04) (width 0.5) (layer "B.Cu") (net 15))
 (segment (start 79 65.5) (end 79 85) (width 0.5) (layer "B.Cu") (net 15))
 (segment (start 116.04 44.5) (end 116.04 45) (width 0.5) (layer "B.Cu") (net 15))
 (segment (start 83.78 89.78) (end 85 89.78) (width 0.5) (layer "B.Cu") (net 15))
 (segment (start 116.04 44.04) (end 116.04 44.5) (width 0.5) (layer "B.Cu") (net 15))
 (segment (start 121 49.96) (end 121 54.5) (width 0.5) (layer "B.Cu") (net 15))
 (segment (start 84 43) (end 115 43) (width 0.5) (layer "B.Cu") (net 15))
 (segment (start 84.66 65.39) (end 79.11 65.39) (width 0.5) (layer "B.Cu") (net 15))
 (segment (start 116.04 45) (end 121 49.96) (width 0.5) (layer "B.Cu") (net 15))
 (segment (start 79 85) (end 83.78 89.78) (width 0.5) (layer "B.Cu") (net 15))
 (segment (start 79 65.5) (end 79 48) (width 0.5) (layer "B.Cu") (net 15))
 (segment (start 86.45 73.09) (end 85 74.54) (width 0.5) (layer "F.Cu") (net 5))
 (segment (start 87 76.54) (end 85 74.54) (width 0.5) (layer "F.Cu") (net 5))
 (segment (start 118.5 85) (end 107.5 96) (width 0.5) (layer "F.Cu") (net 5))
 (segment (start 118.5 64.62) (end 118.5 85) (width 0.5) (layer "F.Cu") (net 5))
 (segment (start 84.66 50.15) (end 86.45 51.94) (width 0.5) (layer "F.Cu") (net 5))
 (segment (start 86.45 51.94) (end 86.45 73.09) (width 0.5) (layer "F.Cu") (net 5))
 (segment (start 131 72.12) (end 121 62.12) (width 0.5) (layer "F.Cu") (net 5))
 (segment (start 87 91) (end 87 76.54) (width 0.5) (layer "F.Cu") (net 5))
 (segment (start 131 77.5) (end 131 72.12) (width 0.5) (layer "F.Cu") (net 5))
 (segment (start 92 96) (end 87 91) (width 0.5) (layer "F.Cu") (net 5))
 (segment (start 121 62.12) (end 118.5 64.62) (width 0.5) (layer "F.Cu") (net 5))
 (segment (start 107.5 96) (end 92 96) (width 0.5) (layer "F.Cu") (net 5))
 (segment (start 105.48 74.54) (end 105.76 74.82) (width 0.5) (layer "B.Cu") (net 29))
 (segment (start 97.7 74.54) (end 105.48 74.54) (width 0.5) (layer "B.Cu") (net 29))
 (segment (start 105.48 72) (end 105.76 72.28) (width 0.5) (layer "B.Cu") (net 28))
 (segment (start 97.7 72) (end 105.48 72) (width 0.5) (layer "B.Cu") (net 28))
 (segment (start 77.3 79.62) (end 77 79.92) (width 0.5) (layer "F.Cu") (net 3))
 (segment (start 85 79.62) (end 77.3 79.62) (width 0.5) (layer "F.Cu") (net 3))
 (segment (start 85 77.08) (end 77.3 77.08) (width 0.5) (layer "F.Cu") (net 4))
 (segment (start 77.3 77.08) (end 77 77.38) (width 0.5) (layer "F.Cu") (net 4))
 (segment (start 84.66 85.04) (end 85 84.7) (width 0.5) (layer "F.Cu") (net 1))
 (segment (start 77.04 85.04) (end 84.66 85.04) (width 0.5) (layer "F.Cu") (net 1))
 (segment (start 77 85) (end 77.04 85.04) (width 0.5) (layer "F.Cu") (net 1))
 (segment (start 85 82.16) (end 77.3 82.16) (width 0.5) (layer "F.Cu") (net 2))
 (segment (start 77.3 82.16) (end 77 82.46) (width 0.5) (layer "F.Cu") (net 2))
 (segment (start 84.39 52.42) (end 84.66 52.69) (width 0.5) (layer "F.Cu") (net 11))
 (segment (start 77 52.42) (end 84.39 52.42) (width 0.5) (layer "F.Cu") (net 11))
 (segment (start 84.39 54.96) (end 84.66 55.23) (width 0.5) (layer "F.Cu") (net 12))
 (segment (start 77 54.96) (end 84.39 54.96) (width 0.5) (layer "F.Cu") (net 12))
 (segment (start 77 57.5) (end 84.39 57.5) (width 0.5) (layer "F.Cu") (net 13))
 (segment (start 84.39 57.5) (end 84.66 57.77) (width 0.5) (layer "F.Cu") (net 13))
 (segment (start 84.39 60.04) (end 84.66 60.31) (width 0.5) (layer "F.Cu") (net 14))
 (segment (start 77 60.04) (end 84.39 60.04) (width 0.5) (layer "F.Cu") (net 14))
 (segment (start 100 64) (end 100 52.79) (width 0.5) (layer "B.Cu") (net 22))
 (segment (start 105.76 69.74) (end 105.74 69.74) (width 0.5) (layer "B.Cu") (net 22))
 (segment (start 100 52.79) (end 97.36 50.15) (width 0.5) (layer "B.Cu") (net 22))
 (segment (start 105.74 69.74) (end 100 64) (width 0.5) (layer "B.Cu") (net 22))
 (segment (start 124.16 94.5) (end 112.74 94.5) (width 0.5) (layer "B.Cu") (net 9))
 (segment (start 131 87.66) (end 124.16 94.5) (width 0.5) (layer "B.Cu") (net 9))
 (segment (start 105.76 87.52) (end 106.02 87.52) (width 0.5) (layer "B.Cu") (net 9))
 (segment (start 112.74 94.5) (end 105.76 87.52) (width 0.5) (layer "B.Cu") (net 9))
 (segment (start 130.86 90.06) (end 121 90.06) (width 0.5) (layer "F.Cu") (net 10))
 (segment (start 131 90.2) (end 130.86 90.06) (width 0.5) (layer "F.Cu") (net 10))
 (segment (start 107.027208 90.06) (end 105.76 90.06) (width 0.5) (layer "B.Cu") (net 8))
 (segment (start 132.5 90.821321) (end 127.921321 95.4) (width 0.5) (layer "B.Cu") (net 8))
 (segment (start 132.5 86.62) (end 132.5 90.821321) (width 0.5) (layer "B.Cu") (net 8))
 (segment (start 127.921321 95.4) (end 112.367208 95.4) (width 0.5) (layer "B.Cu") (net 8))
 (segment (start 112.367208 95.4) (end 107.027208 90.06) (width 0.5) (layer "B.Cu") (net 8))
 (segment (start 131 85.12) (end 132.5 86.62) (width 0.5) (layer "B.Cu") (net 8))
 (segment (start 131 82.58) (end 121.58 92) (width 0.5) (layer "B.Cu") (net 7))
 (segment (start 121.58 92) (end 113 92) (width 0.5) (layer "B.Cu") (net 7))
 (segment (start 105.98 84.98) (end 105.76 84.98) (width 0.5) (layer "B.Cu") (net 7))
 (segment (start 113 92) (end 105.98 84.98) (width 0.5) (layer "B.Cu") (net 7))
 (segment (start 100.9 51.15) (end 100.9 62.34) (width 0.5) (layer "B.Cu") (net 23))
 (segment (start 97.36 47.61) (end 100.9 51.15) (width 0.5) (layer "B.Cu") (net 23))
 (segment (start 100.9 62.34) (end 105.76 67.2) (width 0.5) (layer "B.Cu") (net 23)))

